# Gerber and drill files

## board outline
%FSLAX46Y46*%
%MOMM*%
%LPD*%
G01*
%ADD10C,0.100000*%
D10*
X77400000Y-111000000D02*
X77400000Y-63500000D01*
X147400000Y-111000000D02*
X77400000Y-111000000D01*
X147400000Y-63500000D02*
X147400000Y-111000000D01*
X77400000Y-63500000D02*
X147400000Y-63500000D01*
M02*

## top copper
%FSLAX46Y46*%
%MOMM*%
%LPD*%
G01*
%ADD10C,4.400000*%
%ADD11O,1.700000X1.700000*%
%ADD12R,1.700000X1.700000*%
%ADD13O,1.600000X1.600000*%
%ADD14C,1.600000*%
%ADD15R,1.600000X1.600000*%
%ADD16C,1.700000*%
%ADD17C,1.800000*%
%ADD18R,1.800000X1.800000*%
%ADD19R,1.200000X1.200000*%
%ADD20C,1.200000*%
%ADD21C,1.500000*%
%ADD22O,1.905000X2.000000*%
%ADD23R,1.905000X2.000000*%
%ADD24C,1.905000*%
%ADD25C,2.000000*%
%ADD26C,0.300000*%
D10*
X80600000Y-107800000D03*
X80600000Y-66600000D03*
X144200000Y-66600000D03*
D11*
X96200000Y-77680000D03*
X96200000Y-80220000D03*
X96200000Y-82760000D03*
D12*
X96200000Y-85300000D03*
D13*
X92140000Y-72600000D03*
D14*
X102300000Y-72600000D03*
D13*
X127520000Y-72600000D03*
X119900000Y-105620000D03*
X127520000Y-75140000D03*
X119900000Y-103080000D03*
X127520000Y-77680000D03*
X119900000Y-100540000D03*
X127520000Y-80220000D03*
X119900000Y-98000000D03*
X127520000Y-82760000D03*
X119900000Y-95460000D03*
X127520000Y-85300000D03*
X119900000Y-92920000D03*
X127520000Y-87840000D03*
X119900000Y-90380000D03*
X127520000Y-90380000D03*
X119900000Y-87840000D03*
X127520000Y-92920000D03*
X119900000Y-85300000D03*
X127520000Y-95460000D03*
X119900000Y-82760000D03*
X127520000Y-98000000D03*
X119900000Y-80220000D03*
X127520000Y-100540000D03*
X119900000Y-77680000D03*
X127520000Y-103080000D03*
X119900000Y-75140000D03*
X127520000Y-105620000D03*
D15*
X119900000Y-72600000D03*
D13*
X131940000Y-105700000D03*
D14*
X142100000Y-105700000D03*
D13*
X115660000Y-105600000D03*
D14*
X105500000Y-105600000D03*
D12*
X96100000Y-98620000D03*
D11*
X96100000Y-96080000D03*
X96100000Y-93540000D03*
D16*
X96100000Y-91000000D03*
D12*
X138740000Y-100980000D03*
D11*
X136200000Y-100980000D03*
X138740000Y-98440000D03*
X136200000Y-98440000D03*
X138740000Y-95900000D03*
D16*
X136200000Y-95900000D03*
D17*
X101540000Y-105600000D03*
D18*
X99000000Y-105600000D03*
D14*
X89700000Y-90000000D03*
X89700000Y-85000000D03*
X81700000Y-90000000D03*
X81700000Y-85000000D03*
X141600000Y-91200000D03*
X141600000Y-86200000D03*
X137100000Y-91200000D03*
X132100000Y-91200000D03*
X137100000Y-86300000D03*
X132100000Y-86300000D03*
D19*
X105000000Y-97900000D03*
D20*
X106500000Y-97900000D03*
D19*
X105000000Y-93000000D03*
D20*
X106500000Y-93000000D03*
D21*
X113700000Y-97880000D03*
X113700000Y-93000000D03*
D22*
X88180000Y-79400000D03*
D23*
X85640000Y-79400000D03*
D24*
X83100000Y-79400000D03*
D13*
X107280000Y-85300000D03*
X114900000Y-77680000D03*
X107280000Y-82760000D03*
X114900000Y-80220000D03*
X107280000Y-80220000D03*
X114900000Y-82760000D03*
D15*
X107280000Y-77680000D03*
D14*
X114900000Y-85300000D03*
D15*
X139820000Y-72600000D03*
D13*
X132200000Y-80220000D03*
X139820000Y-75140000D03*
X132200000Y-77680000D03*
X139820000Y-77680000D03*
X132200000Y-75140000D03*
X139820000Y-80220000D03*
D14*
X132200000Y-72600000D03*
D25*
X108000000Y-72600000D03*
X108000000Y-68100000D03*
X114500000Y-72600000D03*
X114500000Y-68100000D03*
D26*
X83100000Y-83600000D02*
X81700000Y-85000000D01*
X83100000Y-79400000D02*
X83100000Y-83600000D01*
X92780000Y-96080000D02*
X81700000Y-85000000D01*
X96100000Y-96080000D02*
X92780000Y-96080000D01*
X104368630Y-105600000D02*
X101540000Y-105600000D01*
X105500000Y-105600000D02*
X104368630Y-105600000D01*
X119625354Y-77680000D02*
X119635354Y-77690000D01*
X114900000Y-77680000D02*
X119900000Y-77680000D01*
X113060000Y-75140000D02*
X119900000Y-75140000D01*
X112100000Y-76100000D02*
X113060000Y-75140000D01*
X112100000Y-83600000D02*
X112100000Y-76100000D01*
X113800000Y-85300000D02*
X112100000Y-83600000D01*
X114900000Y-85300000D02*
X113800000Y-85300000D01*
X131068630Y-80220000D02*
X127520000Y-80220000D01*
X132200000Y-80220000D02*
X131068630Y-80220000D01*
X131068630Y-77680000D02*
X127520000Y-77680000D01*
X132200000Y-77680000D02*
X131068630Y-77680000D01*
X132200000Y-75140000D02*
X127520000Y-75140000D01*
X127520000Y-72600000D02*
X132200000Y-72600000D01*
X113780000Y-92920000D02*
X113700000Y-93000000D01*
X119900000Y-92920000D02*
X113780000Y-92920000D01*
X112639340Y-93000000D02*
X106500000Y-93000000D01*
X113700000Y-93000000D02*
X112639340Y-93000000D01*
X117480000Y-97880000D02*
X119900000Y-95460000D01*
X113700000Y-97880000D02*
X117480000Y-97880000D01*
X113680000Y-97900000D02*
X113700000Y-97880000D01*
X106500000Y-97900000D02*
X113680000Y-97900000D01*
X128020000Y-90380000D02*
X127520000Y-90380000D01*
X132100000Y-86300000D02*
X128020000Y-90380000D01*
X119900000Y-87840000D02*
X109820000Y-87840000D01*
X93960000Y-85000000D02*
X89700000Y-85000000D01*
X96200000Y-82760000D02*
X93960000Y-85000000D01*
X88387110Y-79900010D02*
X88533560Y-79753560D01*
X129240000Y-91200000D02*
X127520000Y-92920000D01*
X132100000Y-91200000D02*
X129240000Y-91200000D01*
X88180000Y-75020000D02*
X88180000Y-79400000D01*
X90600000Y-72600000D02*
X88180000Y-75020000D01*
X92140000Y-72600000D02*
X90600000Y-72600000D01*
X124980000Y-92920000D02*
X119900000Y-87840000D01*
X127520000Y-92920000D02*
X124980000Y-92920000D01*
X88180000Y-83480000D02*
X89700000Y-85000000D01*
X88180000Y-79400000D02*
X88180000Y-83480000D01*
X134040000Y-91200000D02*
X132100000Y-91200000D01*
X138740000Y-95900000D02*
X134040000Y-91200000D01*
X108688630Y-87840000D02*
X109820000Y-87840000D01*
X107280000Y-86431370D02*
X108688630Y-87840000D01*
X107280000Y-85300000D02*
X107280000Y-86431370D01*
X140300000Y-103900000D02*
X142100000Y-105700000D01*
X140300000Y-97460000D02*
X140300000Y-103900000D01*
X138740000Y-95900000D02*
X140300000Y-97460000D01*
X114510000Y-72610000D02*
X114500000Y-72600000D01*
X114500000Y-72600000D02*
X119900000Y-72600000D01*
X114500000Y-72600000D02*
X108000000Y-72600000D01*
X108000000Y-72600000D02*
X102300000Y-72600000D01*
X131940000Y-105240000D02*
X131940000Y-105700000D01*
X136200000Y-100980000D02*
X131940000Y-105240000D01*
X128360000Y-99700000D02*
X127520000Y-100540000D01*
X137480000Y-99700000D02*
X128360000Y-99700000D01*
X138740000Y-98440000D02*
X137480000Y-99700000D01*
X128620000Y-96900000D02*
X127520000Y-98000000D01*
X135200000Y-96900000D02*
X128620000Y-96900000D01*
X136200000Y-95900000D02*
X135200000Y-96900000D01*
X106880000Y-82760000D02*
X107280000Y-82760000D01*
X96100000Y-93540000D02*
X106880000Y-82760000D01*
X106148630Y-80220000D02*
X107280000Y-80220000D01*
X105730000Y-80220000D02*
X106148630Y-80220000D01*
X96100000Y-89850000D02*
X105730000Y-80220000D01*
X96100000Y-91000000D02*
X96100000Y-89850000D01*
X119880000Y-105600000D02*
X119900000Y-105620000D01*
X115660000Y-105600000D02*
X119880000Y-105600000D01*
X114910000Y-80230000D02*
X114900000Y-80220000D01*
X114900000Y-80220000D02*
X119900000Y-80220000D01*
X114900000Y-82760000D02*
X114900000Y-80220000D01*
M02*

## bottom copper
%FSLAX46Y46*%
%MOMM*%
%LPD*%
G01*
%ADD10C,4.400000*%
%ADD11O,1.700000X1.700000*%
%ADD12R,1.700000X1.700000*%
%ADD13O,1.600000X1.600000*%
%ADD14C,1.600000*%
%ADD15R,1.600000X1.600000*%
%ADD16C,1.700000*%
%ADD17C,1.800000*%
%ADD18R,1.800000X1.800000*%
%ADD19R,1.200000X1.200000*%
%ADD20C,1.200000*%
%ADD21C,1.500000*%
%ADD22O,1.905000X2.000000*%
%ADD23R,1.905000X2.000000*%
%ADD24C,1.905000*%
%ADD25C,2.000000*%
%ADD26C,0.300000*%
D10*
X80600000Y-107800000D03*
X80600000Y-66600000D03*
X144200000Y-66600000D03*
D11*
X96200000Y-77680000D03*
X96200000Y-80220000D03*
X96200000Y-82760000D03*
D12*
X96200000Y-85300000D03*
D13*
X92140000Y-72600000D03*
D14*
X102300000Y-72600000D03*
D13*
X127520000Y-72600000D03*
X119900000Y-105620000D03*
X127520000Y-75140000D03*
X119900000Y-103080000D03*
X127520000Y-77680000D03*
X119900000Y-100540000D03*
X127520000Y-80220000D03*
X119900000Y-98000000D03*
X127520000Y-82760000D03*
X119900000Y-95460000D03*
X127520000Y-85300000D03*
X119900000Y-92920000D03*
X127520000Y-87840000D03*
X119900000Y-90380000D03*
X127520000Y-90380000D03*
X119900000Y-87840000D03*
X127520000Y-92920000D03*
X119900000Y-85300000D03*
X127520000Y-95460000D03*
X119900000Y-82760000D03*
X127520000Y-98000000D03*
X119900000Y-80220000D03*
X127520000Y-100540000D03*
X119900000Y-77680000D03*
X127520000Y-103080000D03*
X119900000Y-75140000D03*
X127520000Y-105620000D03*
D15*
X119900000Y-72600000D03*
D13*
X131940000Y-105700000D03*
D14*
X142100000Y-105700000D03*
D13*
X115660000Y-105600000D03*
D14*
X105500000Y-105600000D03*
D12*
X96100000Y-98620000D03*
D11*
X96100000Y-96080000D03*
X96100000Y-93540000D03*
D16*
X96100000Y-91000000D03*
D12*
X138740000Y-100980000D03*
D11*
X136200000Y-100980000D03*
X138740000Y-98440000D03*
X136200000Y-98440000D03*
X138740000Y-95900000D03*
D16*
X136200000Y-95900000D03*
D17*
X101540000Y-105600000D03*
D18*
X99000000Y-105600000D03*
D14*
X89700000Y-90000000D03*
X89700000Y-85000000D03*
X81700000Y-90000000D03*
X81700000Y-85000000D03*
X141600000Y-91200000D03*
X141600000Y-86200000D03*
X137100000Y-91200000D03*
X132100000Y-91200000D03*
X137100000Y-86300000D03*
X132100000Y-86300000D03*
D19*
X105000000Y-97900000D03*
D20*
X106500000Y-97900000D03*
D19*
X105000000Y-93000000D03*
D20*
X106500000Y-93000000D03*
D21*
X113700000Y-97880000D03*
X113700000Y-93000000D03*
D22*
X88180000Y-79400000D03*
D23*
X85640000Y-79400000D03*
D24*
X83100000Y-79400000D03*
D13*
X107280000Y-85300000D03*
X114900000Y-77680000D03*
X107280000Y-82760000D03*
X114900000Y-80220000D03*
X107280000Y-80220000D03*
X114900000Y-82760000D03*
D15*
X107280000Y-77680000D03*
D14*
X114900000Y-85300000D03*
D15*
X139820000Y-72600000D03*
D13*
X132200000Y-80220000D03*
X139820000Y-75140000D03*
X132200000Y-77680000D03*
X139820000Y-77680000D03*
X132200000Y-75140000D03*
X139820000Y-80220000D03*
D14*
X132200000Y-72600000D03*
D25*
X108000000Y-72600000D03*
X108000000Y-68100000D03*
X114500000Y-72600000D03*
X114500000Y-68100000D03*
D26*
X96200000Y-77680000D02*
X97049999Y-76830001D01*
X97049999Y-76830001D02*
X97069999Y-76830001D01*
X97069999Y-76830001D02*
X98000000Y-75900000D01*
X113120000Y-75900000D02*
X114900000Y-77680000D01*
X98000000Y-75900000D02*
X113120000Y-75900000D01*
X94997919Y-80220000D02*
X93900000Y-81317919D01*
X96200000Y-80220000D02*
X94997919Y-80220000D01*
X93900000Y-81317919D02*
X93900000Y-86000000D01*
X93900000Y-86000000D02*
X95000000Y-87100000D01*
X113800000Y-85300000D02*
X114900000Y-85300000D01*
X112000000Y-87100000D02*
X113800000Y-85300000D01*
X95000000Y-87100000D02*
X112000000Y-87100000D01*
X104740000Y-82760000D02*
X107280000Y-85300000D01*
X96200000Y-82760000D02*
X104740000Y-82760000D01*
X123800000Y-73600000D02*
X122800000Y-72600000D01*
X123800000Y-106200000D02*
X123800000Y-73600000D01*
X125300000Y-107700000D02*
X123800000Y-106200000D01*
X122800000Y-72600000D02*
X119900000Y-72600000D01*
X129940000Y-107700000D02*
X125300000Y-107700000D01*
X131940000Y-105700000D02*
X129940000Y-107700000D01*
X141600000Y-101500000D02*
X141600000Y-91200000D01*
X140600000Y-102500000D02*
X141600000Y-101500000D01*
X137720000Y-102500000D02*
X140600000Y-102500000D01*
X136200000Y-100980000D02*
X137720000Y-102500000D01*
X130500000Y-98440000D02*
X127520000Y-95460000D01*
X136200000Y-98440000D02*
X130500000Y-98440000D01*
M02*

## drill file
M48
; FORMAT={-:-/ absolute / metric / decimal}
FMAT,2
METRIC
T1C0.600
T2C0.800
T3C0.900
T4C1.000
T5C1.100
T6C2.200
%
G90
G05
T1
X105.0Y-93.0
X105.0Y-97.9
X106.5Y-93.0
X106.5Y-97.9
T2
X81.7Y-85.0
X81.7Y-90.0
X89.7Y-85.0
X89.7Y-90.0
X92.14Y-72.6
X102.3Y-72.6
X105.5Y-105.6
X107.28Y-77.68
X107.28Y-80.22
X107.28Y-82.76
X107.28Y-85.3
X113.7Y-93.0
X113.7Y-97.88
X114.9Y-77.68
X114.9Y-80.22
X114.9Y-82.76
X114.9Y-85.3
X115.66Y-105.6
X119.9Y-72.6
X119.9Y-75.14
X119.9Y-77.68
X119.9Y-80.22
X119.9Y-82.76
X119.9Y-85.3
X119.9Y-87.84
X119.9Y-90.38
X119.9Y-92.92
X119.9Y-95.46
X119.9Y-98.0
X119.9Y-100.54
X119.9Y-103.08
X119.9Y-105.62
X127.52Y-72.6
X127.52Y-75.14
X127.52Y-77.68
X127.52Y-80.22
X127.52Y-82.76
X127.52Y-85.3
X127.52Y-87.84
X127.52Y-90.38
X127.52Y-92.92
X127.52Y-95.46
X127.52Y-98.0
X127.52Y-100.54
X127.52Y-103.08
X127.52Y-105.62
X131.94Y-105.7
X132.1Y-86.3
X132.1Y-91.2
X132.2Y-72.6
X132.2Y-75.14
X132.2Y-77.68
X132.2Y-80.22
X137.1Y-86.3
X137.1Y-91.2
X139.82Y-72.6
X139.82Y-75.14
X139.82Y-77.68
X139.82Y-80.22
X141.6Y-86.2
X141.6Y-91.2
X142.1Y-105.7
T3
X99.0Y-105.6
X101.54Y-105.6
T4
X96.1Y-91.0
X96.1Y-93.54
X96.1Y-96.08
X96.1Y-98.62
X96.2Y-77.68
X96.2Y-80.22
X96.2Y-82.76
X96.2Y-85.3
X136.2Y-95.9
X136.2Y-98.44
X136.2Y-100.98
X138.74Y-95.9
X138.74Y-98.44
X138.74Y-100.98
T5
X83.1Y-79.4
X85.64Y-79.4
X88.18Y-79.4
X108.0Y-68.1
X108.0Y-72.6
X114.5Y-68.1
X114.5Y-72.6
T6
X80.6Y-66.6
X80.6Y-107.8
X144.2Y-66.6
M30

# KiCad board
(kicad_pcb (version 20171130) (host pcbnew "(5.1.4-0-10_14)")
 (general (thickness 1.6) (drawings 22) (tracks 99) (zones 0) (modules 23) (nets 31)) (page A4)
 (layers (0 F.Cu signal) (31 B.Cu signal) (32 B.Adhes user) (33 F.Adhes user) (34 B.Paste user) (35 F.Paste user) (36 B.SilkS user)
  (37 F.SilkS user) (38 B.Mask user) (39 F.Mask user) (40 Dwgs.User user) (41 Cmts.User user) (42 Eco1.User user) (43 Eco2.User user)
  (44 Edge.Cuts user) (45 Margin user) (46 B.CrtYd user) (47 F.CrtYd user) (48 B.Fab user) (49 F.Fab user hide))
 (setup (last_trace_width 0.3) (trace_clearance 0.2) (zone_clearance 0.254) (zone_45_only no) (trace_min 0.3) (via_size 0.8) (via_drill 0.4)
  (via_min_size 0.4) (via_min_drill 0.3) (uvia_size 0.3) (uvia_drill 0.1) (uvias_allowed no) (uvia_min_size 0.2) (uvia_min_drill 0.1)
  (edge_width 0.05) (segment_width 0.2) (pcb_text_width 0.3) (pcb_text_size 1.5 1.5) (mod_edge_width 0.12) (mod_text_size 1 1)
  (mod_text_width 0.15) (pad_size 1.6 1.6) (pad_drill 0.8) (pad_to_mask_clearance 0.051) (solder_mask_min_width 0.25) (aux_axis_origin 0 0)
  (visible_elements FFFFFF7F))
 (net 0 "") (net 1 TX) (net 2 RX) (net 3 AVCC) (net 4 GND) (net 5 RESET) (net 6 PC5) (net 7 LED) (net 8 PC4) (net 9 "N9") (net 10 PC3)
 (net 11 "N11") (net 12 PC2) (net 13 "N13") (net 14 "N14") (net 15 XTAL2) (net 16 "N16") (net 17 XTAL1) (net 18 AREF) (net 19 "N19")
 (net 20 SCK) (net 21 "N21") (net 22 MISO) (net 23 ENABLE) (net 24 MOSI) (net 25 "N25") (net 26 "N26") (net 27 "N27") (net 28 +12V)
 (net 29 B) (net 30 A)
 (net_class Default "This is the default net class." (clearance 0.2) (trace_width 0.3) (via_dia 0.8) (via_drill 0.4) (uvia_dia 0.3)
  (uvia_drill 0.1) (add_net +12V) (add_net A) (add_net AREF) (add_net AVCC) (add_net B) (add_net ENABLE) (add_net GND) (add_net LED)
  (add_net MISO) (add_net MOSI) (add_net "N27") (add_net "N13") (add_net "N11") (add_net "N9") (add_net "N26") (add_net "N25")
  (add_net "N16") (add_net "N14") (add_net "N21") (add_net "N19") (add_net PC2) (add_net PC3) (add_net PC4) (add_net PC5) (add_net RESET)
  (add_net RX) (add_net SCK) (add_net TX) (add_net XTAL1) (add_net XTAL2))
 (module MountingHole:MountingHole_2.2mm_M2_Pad (layer F.Cu) (at 80.6 107.8)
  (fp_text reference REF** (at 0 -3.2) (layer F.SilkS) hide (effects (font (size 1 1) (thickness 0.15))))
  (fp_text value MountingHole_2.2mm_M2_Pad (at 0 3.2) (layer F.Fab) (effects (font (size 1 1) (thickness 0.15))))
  (pad 1 thru_hole circle (at 0 0) (size 4.4 4.4) (drill 2.2) (layers *.Cu *.Mask)))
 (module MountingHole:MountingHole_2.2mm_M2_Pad (layer F.Cu) (at 80.6 66.6)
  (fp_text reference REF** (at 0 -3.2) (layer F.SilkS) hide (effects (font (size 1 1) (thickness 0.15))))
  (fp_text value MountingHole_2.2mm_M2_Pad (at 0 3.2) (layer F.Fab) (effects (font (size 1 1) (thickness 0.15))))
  (pad 1 thru_hole circle (at 0 0) (size 4.4 4.4) (drill 2.2) (layers *.Cu *.Mask)))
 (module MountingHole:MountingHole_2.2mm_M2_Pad (layer F.Cu) (at 144.2 66.6)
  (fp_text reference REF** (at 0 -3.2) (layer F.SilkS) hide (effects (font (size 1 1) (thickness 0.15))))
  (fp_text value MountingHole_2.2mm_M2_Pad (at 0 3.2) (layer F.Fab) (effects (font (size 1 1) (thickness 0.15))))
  (pad 1 thru_hole circle (at 0 0) (size 4.4 4.4) (drill 2.2) (layers *.Cu *.Mask)))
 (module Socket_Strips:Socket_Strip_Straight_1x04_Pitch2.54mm (layer F.Cu) (at 96.2 85.3 180)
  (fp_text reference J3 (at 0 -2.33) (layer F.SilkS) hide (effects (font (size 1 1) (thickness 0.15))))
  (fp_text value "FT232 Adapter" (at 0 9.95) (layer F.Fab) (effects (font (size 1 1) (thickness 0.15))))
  (pad 4 thru_hole oval (at 0 7.62 180) (size 1.7 1.7) (drill 1) (layers *.Cu *.Mask) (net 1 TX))
  (pad 3 thru_hole oval (at 0 5.08 180) (size 1.7 1.7) (drill 1) (layers *.Cu *.Mask) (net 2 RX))
  (pad 2 thru_hole oval (at 0 2.54 180) (size 1.7 1.7) (drill 1) (layers *.Cu *.Mask) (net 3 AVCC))
  (pad 1 thru_hole rect (at 0 0 180) (size 1.7 1.7) (drill 1) (layers *.Cu *.Mask) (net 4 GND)))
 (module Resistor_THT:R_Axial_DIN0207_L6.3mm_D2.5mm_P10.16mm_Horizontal (layer F.Cu) (at 102.3 72.6 180)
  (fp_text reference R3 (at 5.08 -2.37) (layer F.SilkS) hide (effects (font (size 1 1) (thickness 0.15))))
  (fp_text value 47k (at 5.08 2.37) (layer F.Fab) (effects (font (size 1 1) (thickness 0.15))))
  (pad 2 thru_hole oval (at 10.16 0 180) (size 1.6 1.6) (drill 0.8) (layers *.Cu *.Mask) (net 3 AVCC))
  (pad 1 thru_hole circle (at 0 0 180) (size 1.6 1.6) (drill 0.8) (layers *.Cu *.Mask) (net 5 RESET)))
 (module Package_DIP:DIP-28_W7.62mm (layer F.Cu) (at 119.9 72.6)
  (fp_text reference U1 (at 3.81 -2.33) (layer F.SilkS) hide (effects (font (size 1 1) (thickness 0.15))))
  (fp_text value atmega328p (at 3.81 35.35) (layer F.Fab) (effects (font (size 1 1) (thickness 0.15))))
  (pad 28 thru_hole oval (at 7.62 0) (size 1.6 1.6) (drill 0.8) (layers *.Cu *.Mask) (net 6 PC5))
  (pad 14 thru_hole oval (at 0 33.02) (size 1.6 1.6) (drill 0.8) (layers *.Cu *.Mask) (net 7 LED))
  (pad 27 thru_hole oval (at 7.62 2.54) (size 1.6 1.6) (drill 0.8) (layers *.Cu *.Mask) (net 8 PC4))
  (pad 13 thru_hole oval (at 0 30.48) (size 1.6 1.6) (drill 0.8) (layers *.Cu *.Mask) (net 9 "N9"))
  (pad 26 thru_hole oval (at 7.62 5.08) (size 1.6 1.6) (drill 0.8) (layers *.Cu *.Mask) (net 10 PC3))
  (pad 12 thru_hole oval (at 0 27.94) (size 1.6 1.6) (drill 0.8) (layers *.Cu *.Mask) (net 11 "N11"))
  (pad 25 thru_hole oval (at 7.62 7.62) (size 1.6 1.6) (drill 0.8) (layers *.Cu *.Mask) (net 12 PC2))
  (pad 11 thru_hole oval (at 0 25.4) (size 1.6 1.6) (drill 0.8) (layers *.Cu *.Mask) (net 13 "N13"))
  (pad 24 thru_hole oval (at 7.62 10.16) (size 1.6 1.6) (drill 0.8) (layers *.Cu *.Mask) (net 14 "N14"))
  (pad 10 thru_hole oval (at 0 22.86) (size 1.6 1.6) (drill 0.8) (layers *.Cu *.Mask) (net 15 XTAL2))
  (pad 23 thru_hole oval (at 7.62 12.7) (size 1.6 1.6) (drill 0.8) (layers *.Cu *.Mask) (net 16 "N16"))
  (pad 9 thru_hole oval (at 0 20.32) (size 1.6 1.6) (drill 0.8) (layers *.Cu *.Mask) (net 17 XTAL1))
  (pad 22 thru_hole oval (at 7.62 15.24) (size 1.6 1.6) (drill 0.8) (layers *.Cu *.Mask) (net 4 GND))
  (pad 8 thru_hole oval (at 0 17.78) (size 1.6 1.6) (drill 0.8) (layers *.Cu *.Mask) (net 4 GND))
  (pad 21 thru_hole oval (at 7.62 17.78) (size 1.6 1.6) (drill 0.8) (layers *.Cu *.Mask) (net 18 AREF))
  (pad 7 thru_hole oval (at 0 15.24) (size 1.6 1.6) (drill 0.8) (layers *.Cu *.Mask) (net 3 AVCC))
  (pad 20 thru_hole oval (at 7.62 20.32) (size 1.6 1.6) (drill 0.8) (layers *.Cu *.Mask) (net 3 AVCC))
  (pad 6 thru_hole oval (at 0 12.7) (size 1.6 1.6) (drill 0.8) (layers *.Cu *.Mask) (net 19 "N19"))
  (pad 19 thru_hole oval (at 7.62 22.86) (size 1.6 1.6) (drill 0.8) (layers *.Cu *.Mask) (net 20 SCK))
  (pad 5 thru_hole oval (at 0 10.16) (size 1.6 1.6) (drill 0.8) (layers *.Cu *.Mask) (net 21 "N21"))
  (pad 18 thru_hole oval (at 7.62 25.4) (size 1.6 1.6) (drill 0.8) (layers *.Cu *.Mask) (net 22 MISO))
  (pad 4 thru_hole oval (at 0 7.62) (size 1.6 1.6) (drill 0.8) (layers *.Cu *.Mask) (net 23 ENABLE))
  (pad 17 thru_hole oval (at 7.62 27.94) (size 1.6 1.6) (drill 0.8) (layers *.Cu *.Mask) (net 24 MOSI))
  (pad 3 thru_hole oval (at 0 5.08) (size 1.6 1.6) (drill 0.8) (layers *.Cu *.Mask) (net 1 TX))
  (pad 16 thru_hole oval (at 7.62 30.48) (size 1.6 1.6) (drill 0.8) (layers *.Cu *.Mask) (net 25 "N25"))
  (pad 2 thru_hole oval (at 0 2.54) (size 1.6 1.6) (drill 0.8) (layers *.Cu *.Mask) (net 2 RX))
  (pad 15 thru_hole oval (at 7.62 33.02) (size 1.6 1.6) (drill 0.8) (layers *.Cu *.Mask) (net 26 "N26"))
  (pad 1 thru_hole rect (at 0 0) (size 1.6 1.6) (drill 0.8) (layers *.Cu *.Mask) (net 5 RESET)))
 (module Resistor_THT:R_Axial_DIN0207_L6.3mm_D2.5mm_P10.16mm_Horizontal (layer F.Cu) (at 142.1 105.7 180)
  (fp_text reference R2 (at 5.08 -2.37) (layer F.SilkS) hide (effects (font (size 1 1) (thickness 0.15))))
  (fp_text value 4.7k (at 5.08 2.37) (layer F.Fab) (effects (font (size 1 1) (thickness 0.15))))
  (pad 2 thru_hole oval (at 10.16 0 180) (size 1.6 1.6) (drill 0.8) (layers *.Cu *.Mask) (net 5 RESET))
  (pad 1 thru_hole circle (at 0 0 180) (size 1.6 1.6) (drill 0.8) (layers *.Cu *.Mask) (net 3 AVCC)))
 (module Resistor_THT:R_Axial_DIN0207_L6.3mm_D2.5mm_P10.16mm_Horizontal (layer F.Cu) (at 105.5 105.6)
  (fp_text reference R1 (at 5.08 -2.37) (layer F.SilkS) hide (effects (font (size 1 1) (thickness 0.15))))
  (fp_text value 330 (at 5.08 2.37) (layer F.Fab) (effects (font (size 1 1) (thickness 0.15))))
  (pad 2 thru_hole oval (at 10.16 0) (size 1.6 1.6) (drill 0.8) (layers *.Cu *.Mask) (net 7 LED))
  (pad 1 thru_hole circle (at 0 0) (size 1.6 1.6) (drill 0.8) (layers *.Cu *.Mask) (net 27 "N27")))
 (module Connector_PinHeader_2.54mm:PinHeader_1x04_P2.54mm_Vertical (layer F.Cu) (at 96.1 91)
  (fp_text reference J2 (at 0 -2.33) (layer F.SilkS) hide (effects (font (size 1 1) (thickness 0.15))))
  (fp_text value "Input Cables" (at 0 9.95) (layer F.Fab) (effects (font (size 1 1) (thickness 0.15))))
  (pad 4 thru_hole rect (at 0 7.62) (size 1.7 1.7) (drill 1) (layers *.Cu *.Mask) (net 4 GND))
  (pad 3 thru_hole oval (at 0 5.08) (size 1.7 1.7) (drill 1) (layers *.Cu *.Mask) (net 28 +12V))
  (pad 2 thru_hole oval (at 0 2.54) (size 1.7 1.7) (drill 1) (layers *.Cu *.Mask) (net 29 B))
  (pad 1 thru_hole circle (at 0 0) (size 1.7 1.7) (drill 1) (layers *.Cu *.Mask) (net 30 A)))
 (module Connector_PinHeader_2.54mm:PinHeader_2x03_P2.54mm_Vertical (layer F.Cu) (at 136.2 95.9)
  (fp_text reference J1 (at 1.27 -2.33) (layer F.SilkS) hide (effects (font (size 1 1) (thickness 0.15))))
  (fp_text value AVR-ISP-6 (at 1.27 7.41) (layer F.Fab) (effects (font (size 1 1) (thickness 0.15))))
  (pad 6 thru_hole rect (at 2.54 5.08) (size 1.7 1.7) (drill 1) (layers *.Cu *.Mask) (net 4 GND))
  (pad 5 thru_hole oval (at 0 5.08) (size 1.7 1.7) (drill 1) (layers *.Cu *.Mask) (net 5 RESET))
  (pad 4 thru_hole oval (at 2.54 2.54) (size 1.7 1.7) (drill 1) (layers *.Cu *.Mask) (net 24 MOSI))
  (pad 3 thru_hole oval (at 0 2.54) (size 1.7 1.7) (drill 1) (layers *.Cu *.Mask) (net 20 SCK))
  (pad 2 thru_hole oval (at 2.54 0) (size 1.7 1.7) (drill 1) (layers *.Cu *.Mask) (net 3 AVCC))
  (pad 1 thru_hole circle (at 0 0) (size 1.7 1.7) (drill 1) (layers *.Cu *.Mask) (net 22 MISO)))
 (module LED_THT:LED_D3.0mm (layer F.Cu) (at 99 105.6)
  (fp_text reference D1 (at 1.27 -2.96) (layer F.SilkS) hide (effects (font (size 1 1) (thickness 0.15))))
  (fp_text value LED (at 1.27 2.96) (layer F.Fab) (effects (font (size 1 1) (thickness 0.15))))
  (pad 2 thru_hole circle (at 2.54 0) (size 1.8 1.8) (drill 0.9) (layers *.Cu *.Mask) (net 27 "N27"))
  (pad 1 thru_hole rect (at 0 0) (size 1.8 1.8) (drill 0.9) (layers *.Cu *.Mask) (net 4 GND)))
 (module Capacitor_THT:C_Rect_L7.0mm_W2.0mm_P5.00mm (layer F.Cu) (at 89.7 85 270)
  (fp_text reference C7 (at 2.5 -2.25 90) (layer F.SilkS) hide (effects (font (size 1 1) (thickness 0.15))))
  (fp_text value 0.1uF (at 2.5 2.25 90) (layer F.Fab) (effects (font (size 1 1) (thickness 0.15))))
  (pad 2 thru_hole circle (at 5 0 270) (size 1.6 1.6) (drill 0.8) (layers *.Cu *.Mask) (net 4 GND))
  (pad 1 thru_hole circle (at 0 0 270) (size 1.6 1.6) (drill 0.8) (layers *.Cu *.Mask) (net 3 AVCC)))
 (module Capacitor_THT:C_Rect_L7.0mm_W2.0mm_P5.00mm (layer F.Cu) (at 81.7 85 270)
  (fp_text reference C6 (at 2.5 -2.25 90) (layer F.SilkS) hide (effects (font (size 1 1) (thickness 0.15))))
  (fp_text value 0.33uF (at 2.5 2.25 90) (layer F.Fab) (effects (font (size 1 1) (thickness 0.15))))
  (pad 2 thru_hole circle (at 5 0 270) (size 1.6 1.6) (drill 0.8) (layers *.Cu *.Mask) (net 4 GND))
  (pad 1 thru_hole circle (at 0 0 270) (size 1.6 1.6) (drill 0.8) (layers *.Cu *.Mask) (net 28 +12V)))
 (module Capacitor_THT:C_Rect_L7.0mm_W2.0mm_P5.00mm (layer F.Cu) (at 141.6 86.2 270)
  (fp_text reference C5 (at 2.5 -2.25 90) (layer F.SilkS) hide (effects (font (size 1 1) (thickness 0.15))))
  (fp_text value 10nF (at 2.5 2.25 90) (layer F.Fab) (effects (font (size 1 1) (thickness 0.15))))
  (pad 2 thru_hole circle (at 5 0 270) (size 1.6 1.6) (drill 0.8) (layers *.Cu *.Mask) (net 5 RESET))
  (pad 1 thru_hole circle (at 0 0 270) (size 1.6 1.6) (drill 0.8) (layers *.Cu *.Mask) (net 4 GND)))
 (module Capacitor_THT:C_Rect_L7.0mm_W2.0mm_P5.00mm (layer F.Cu) (at 132.1 91.2)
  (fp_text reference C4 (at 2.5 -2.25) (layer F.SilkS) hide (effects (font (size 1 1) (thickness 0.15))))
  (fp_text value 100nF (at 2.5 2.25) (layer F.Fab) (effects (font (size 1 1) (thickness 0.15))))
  (pad 2 thru_hole circle (at 5 0) (size 1.6 1.6) (drill 0.8) (layers *.Cu *.Mask) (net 4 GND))
  (pad 1 thru_hole circle (at 0 0) (size 1.6 1.6) (drill 0.8) (layers *.Cu *.Mask) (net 3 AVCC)))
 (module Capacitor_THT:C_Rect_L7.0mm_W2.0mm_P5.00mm (layer F.Cu) (at 132.1 86.3)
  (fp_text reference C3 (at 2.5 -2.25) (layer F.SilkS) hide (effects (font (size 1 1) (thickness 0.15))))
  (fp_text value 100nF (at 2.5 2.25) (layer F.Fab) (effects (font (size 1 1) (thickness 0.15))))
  (pad 2 thru_hole circle (at 5 0) (size 1.6 1.6) (drill 0.8) (layers *.Cu *.Mask) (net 4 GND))
  (pad 1 thru_hole circle (at 0 0) (size 1.6 1.6) (drill 0.8) (layers *.Cu *.Mask) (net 18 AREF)))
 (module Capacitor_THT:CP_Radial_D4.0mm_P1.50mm (layer F.Cu) (at 106.5 97.9 180)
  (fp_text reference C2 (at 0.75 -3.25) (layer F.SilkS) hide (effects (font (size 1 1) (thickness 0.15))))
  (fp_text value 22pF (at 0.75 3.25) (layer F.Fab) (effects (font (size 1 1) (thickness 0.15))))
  (pad 2 thru_hole rect (at 1.5 0 180) (size 1.2 1.2) (drill 0.6) (layers *.Cu *.Mask) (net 4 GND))
  (pad 1 thru_hole circle (at 0 0 180) (size 1.2 1.2) (drill 0.6) (layers *.Cu *.Mask) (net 15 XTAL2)))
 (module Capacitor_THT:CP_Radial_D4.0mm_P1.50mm (layer F.Cu) (at 106.5 93 180)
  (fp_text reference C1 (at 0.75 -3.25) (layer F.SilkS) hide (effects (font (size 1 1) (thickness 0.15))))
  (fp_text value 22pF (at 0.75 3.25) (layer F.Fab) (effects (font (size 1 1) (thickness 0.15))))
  (pad 2 thru_hole rect (at 1.5 0 180) (size 1.2 1.2) (drill 0.6) (layers *.Cu *.Mask) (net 4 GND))
  (pad 1 thru_hole circle (at 0 0 180) (size 1.2 1.2) (drill 0.6) (layers *.Cu *.Mask) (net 17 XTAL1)))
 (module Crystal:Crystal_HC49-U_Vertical (layer F.Cu) (at 113.7 93 270)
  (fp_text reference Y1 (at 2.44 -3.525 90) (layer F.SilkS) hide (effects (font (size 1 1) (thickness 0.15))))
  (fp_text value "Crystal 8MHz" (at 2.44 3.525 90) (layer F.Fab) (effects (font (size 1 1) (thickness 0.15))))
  (pad 2 thru_hole circle (at 4.88 0 270) (size 1.5 1.5) (drill 0.8) (layers *.Cu *.Mask) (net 15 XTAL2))
  (pad 1 thru_hole circle (at 0 0 270) (size 1.5 1.5) (drill 0.8) (layers *.Cu *.Mask) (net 17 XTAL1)))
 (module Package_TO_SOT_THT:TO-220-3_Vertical (layer F.Cu) (at 83.1 79.4)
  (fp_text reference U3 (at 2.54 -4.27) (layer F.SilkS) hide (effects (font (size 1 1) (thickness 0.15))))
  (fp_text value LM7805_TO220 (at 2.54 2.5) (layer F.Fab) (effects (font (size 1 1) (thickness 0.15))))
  (pad 3 thru_hole oval (at 5.08 0) (size 1.905 2) (drill 1.1) (layers *.Cu *.Mask) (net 3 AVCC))
  (pad 2 thru_hole rect (at 2.54 0) (size 1.905 2) (drill 1.1) (layers *.Cu *.Mask) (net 4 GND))
  (pad 1 thru_hole circle (at 0 0) (size 1.905 1.905) (drill 1.1) (layers *.Cu *.Mask) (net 28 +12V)))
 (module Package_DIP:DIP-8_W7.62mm (layer F.Cu) (at 114.9 85.3 180)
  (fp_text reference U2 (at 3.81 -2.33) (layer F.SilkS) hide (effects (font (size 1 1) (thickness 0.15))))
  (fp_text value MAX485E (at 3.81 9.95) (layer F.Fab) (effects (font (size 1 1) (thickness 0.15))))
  (pad 8 thru_hole oval (at 7.62 0 180) (size 1.6 1.6) (drill 0.8) (layers *.Cu *.Mask) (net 3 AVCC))
  (pad 4 thru_hole oval (at 0 7.62 180) (size 1.6 1.6) (drill 0.8) (layers *.Cu *.Mask) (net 1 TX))
  (pad 7 thru_hole oval (at 7.62 2.54 180) (size 1.6 1.6) (drill 0.8) (layers *.Cu *.Mask) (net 29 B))
  (pad 3 thru_hole oval (at 0 5.08 180) (size 1.6 1.6) (drill 0.8) (layers *.Cu *.Mask) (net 23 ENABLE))
  (pad 6 thru_hole oval (at 7.62 5.08 180) (size 1.6 1.6) (drill 0.8) (layers *.Cu *.Mask) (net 30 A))
  (pad 2 thru_hole oval (at 0 2.54 180) (size 1.6 1.6) (drill 0.8) (layers *.Cu *.Mask) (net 23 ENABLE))
  (pad 5 thru_hole rect (at 7.62 7.62 180) (size 1.6 1.6) (drill 0.8) (layers *.Cu *.Mask) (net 4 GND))
  (pad 1 thru_hole circle (at 0 0 180) (size 1.6 1.6) (drill 0.8) (layers *.Cu *.Mask) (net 2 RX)))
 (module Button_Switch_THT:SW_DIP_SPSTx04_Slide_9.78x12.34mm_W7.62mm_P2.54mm (layer F.Cu) (at 132.2 72.6)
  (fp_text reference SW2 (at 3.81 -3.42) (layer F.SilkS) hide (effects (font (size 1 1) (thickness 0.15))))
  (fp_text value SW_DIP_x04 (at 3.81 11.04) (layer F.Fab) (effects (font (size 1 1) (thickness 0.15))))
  (pad 8 thru_hole rect (at 7.62 0) (size 1.6 1.6) (drill 0.8) (layers *.Cu *.Mask) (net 4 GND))
  (pad 4 thru_hole oval (at 0 7.62) (size 1.6 1.6) (drill 0.8) (layers *.Cu *.Mask) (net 12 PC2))
  (pad 7 thru_hole oval (at 7.62 2.54) (size 1.6 1.6) (drill 0.8) (layers *.Cu *.Mask) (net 4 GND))
  (pad 3 thru_hole oval (at 0 5.08) (size 1.6 1.6) (drill 0.8) (layers *.Cu *.Mask) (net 10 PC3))
  (pad 6 thru_hole oval (at 7.62 5.08) (size 1.6 1.6) (drill 0.8) (layers *.Cu *.Mask) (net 4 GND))
  (pad 2 thru_hole oval (at 0 2.54) (size 1.6 1.6) (drill 0.8) (layers *.Cu *.Mask) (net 8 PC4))
  (pad 5 thru_hole oval (at 7.62 7.62) (size 1.6 1.6) (drill 0.8) (layers *.Cu *.Mask) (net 4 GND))
  (pad 1 thru_hole circle (at 0 0) (size 1.6 1.6) (drill 0.8) (layers *.Cu *.Mask) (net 6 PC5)))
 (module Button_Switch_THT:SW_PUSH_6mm (layer F.Cu) (at 114.5 72.6 180)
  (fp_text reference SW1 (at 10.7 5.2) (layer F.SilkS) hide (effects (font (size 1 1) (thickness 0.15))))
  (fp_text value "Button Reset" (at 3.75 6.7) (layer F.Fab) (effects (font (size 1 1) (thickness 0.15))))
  (pad 1 thru_hole circle (at 6.5 0 270) (size 2 2) (drill 1.1) (layers *.Cu *.Mask) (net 5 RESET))
  (pad 2 thru_hole circle (at 6.5 4.5 270) (size 2 2) (drill 1.1) (layers *.Cu *.Mask) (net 4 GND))
  (pad 1 thru_hole circle (at 0 0 270) (size 2 2) (drill 1.1) (layers *.Cu *.Mask) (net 5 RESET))
  (pad 2 thru_hole circle (at 0 4.5 270) (size 2 2) (drill 1.1) (layers *.Cu *.Mask) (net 4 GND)))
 (gr_line (start 77.4 111) (end 77.4 63.5) (layer Edge.Cuts) (width 0.1))
 (gr_line (start 147.4 111) (end 77.4 111) (layer Edge.Cuts) (width 0.1))
 (gr_line (start 147.4 63.5) (end 147.4 111) (layer Edge.Cuts) (width 0.1))
 (gr_line (start 77.4 63.5) (end 147.4 63.5) (layer Edge.Cuts) (width 0.1))
 (segment (start 83.1 83.6) (end 81.7 85) (width 0.3) (layer F.Cu) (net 28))
 (segment (start 83.1 79.4) (end 83.1 83.6) (width 0.3) (layer F.Cu) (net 28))
 (segment (start 92.78 96.08) (end 81.7 85) (width 0.3) (layer F.Cu) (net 28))
 (segment (start 96.1 96.08) (end 92.78 96.08) (width 0.3) (layer F.Cu) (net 28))
 (segment (start 104.36863 105.6) (end 101.54 105.6) (width 0.3) (layer F.Cu) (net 27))
 (segment (start 105.5 105.6) (end 104.36863 105.6) (width 0.3) (layer F.Cu) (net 27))
 (segment (start 119.625354 77.68) (end 119.635354 77.69) (width 0.3) (layer F.Cu) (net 1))
 (segment (start 114.9 77.68) (end 119.9 77.68) (width 0.3) (layer F.Cu) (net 1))
 (segment (start 96.2 77.68) (end 97.049999 76.830001) (width 0.3) (layer B.Cu) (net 1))
 (segment (start 97.049999 76.830001) (end 97.069999 76.830001) (width 0.3) (layer B.Cu) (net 1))
 (segment (start 97.069999 76.830001) (end 98 75.9) (width 0.3) (layer B.Cu) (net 1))
 (segment (start 113.12 75.9) (end 114.9 77.68) (width 0.3) (layer B.Cu) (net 1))
 (segment (start 98 75.9) (end 113.12 75.9) (width 0.3) (layer B.Cu) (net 1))
 (segment (start 113.06 75.14) (end 119.9 75.14) (width 0.3) (layer F.Cu) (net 2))
 (segment (start 112.1 76.1) (end 113.06 75.14) (width 0.3) (layer F.Cu) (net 2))
 (segment (start 112.1 83.6) (end 112.1 76.1) (width 0.3) (layer F.Cu) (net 2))
 (segment (start 113.8 85.3) (end 112.1 83.6) (width 0.3) (layer F.Cu) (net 2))
 (segment (start 114.9 85.3) (end 113.8 85.3) (width 0.3) (layer F.Cu) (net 2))
 (segment (start 94.997919 80.22) (end 93.9 81.317919) (width 0.3) (layer B.Cu) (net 2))
 (segment (start 96.2 80.22) (end 94.997919 80.22) (width 0.3) (layer B.Cu) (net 2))
 (segment (start 93.9 81.317919) (end 93.9 86) (width 0.3) (layer B.Cu) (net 2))
 (segment (start 93.9 86) (end 95 87.1) (width 0.3) (layer B.Cu) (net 2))
 (segment (start 113.8 85.3) (end 114.9 85.3) (width 0.3) (layer B.Cu) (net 2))
 (segment (start 112 87.1) (end 113.8 85.3) (width 0.3) (layer B.Cu) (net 2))
 (segment (start 95 87.1) (end 112 87.1) (width 0.3) (layer B.Cu) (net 2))
 (segment (start 131.06863 80.22) (end 127.52 80.22) (width 0.3) (layer F.Cu) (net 12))
 (segment (start 132.2 80.22) (end 131.06863 80.22) (width 0.3) (layer F.Cu) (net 12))
 (segment (start 131.06863 77.68) (end 127.52 77.68) (width 0.3) (layer F.Cu) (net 10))
 (segment (start 132.2 77.68) (end 131.06863 77.68) (width 0.3) (layer F.Cu) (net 10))
 (segment (start 132.2 75.14) (end 127.52 75.14) (width 0.3) (layer F.Cu) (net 8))
 (segment (start 127.52 72.6) (end 132.2 72.6) (width 0.3) (layer F.Cu) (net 6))
 (segment (start 113.78 92.92) (end 113.7 93) (width 0.3) (layer F.Cu) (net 17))
 (segment (start 119.9 92.92) (end 113.78 92.92) (width 0.3) (layer F.Cu) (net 17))
 (segment (start 112.63934 93) (end 106.5 93) (width 0.3) (layer F.Cu) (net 17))
 (segment (start 113.7 93) (end 112.63934 93) (width 0.3) (layer F.Cu) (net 17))
 (segment (start 117.48 97.88) (end 119.9 95.46) (width 0.3) (layer F.Cu) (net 15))
 (segment (start 113.7 97.88) (end 117.48 97.88) (width 0.3) (layer F.Cu) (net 15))
 (segment (start 113.68 97.9) (end 113.7 97.88) (width 0.3) (layer F.Cu) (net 15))
 (segment (start 106.5 97.9) (end 113.68 97.9) (width 0.3) (layer F.Cu) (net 15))
 (segment (start 128.02 90.38) (end 127.52 90.38) (width 0.3) (layer F.Cu) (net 18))
 (segment (start 132.1 86.3) (end 128.02 90.38) (width 0.3) (layer F.Cu) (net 18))
 (segment (start 119.9 87.84) (end 109.82 87.84) (width 0.3) (layer F.Cu) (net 3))
 (segment (start 93.96 85) (end 89.7 85) (width 0.3) (layer F.Cu) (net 3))
 (segment (start 96.2 82.76) (end 93.96 85) (width 0.3) (layer F.Cu) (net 3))
 (segment (start 88.38711 79.90001) (end 88.53356 79.75356) (width 0.3) (layer F.Cu) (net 3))
 (segment (start 129.24 91.2) (end 127.52 92.92) (width 0.3) (layer F.Cu) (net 3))
 (segment (start 132.1 91.2) (end 129.24 91.2) (width 0.3) (layer F.Cu) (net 3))
 (segment (start 88.18 75.02) (end 88.18 79.4) (width 0.3) (layer F.Cu) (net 3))
 (segment (start 90.6 72.6) (end 88.18 75.02) (width 0.3) (layer F.Cu) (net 3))
 (segment (start 92.14 72.6) (end 90.6 72.6) (width 0.3) (layer F.Cu) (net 3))
 (segment (start 124.98 92.92) (end 119.9 87.84) (width 0.3) (layer F.Cu) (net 3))
 (segment (start 127.52 92.92) (end 124.98 92.92) (width 0.3) (layer F.Cu) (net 3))
 (segment (start 104.74 82.76) (end 107.28 85.3) (width 0.3) (layer B.Cu) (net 3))
 (segment (start 96.2 82.76) (end 104.74 82.76) (width 0.3) (layer B.Cu) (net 3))
 (segment (start 88.18 83.48) (end 89.7 85) (width 0.3) (layer F.Cu) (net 3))
 (segment (start 88.18 79.4) (end 88.18 83.48) (width 0.3) (layer F.Cu) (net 3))
 (segment (start 134.04 91.2) (end 132.1 91.2) (width 0.3) (layer F.Cu) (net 3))
 (segment (start 138.74 95.9) (end 134.04 91.2) (width 0.3) (layer F.Cu) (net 3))
 (segment (start 108.68863 87.84) (end 109.82 87.84) (width 0.3) (layer F.Cu) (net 3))
 (segment (start 107.28 86.43137) (end 108.68863 87.84) (width 0.3) (layer F.Cu) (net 3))
 (segment (start 107.28 85.3) (end 107.28 86.43137) (width 0.3) (layer F.Cu) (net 3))
 (segment (start 140.3 103.9) (end 142.1 105.7) (width 0.3) (layer F.Cu) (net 3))
 (segment (start 140.3 97.46) (end 140.3 103.9) (width 0.3) (layer F.Cu) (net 3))
 (segment (start 138.74 95.9) (end 140.3 97.46) (width 0.3) (layer F.Cu) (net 3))
 (segment (start 114.51 72.61) (end 114.5 72.6) (width 0.3) (layer F.Cu) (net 5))
 (segment (start 114.5 72.6) (end 119.9 72.6) (width 0.3) (layer F.Cu) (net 5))
 (segment (start 114.5 72.6) (end 108 72.6) (width 0.3) (layer F.Cu) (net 5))
 (segment (start 108 72.6) (end 102.3 72.6) (width 0.3) (layer F.Cu) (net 5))
 (segment (start 123.8 73.6) (end 122.8 72.6) (width 0.3) (layer B.Cu) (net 5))
 (segment (start 123.8 106.2) (end 123.8 73.6) (width 0.3) (layer B.Cu) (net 5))
 (segment (start 125.3 107.7) (end 123.8 106.2) (width 0.3) (layer B.Cu) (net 5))
 (segment (start 122.8 72.6) (end 119.9 72.6) (width 0.3) (layer B.Cu) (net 5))
 (segment (start 131.94 105.24) (end 131.94 105.7) (width 0.3) (layer F.Cu) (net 5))
 (segment (start 136.2 100.98) (end 131.94 105.24) (width 0.3) (layer F.Cu) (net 5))
 (segment (start 129.94 107.7) (end 125.3 107.7) (width 0.3) (layer B.Cu) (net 5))
 (segment (start 131.94 105.7) (end 129.94 107.7) (width 0.3) (layer B.Cu) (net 5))
 (segment (start 141.6 101.5) (end 141.6 91.2) (width 0.3) (layer B.Cu) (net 5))
 (segment (start 140.6 102.5) (end 141.6 101.5) (width 0.3) (layer B.Cu) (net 5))
 (segment (start 137.72 102.5) (end 140.6 102.5) (width 0.3) (layer B.Cu) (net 5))
 (segment (start 136.2 100.98) (end 137.72 102.5) (width 0.3) (layer B.Cu) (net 5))
 (segment (start 128.36 99.7) (end 127.52 100.54) (width 0.3) (layer F.Cu) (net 24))
 (segment (start 137.48 99.7) (end 128.36 99.7) (width 0.3) (layer F.Cu) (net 24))
 (segment (start 138.74 98.44) (end 137.48 99.7) (width 0.3) (layer F.Cu) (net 24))
 (segment (start 130.5 98.44) (end 127.52 95.46) (width 0.3) (layer B.Cu) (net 20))
 (segment (start 136.2 98.44) (end 130.5 98.44) (width 0.3) (layer B.Cu) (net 20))
 (segment (start 128.62 96.9) (end 127.52 98) (width 0.3) (layer F.Cu) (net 22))
 (segment (start 135.2 96.9) (end 128.62 96.9) (width 0.3) (layer F.Cu) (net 22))
 (segment (start 136.2 95.9) (end 135.2 96.9) (width 0.3) (layer F.Cu) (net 22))
 (segment (start 106.88 82.76) (end 107.28 82.76) (width 0.3) (layer F.Cu) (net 29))
 (segment (start 96.1 93.54) (end 106.88 82.76) (width 0.3) (layer F.Cu) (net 29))
 (segment (start 106.14863 80.22) (end 107.28 80.22) (width 0.3) (layer F.Cu) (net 30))
 (segment (start 105.73 80.22) (end 106.14863 80.22) (width 0.3) (layer F.Cu) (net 30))
 (segment (start 96.1 89.85) (end 105.73 80.22) (width 0.3) (layer F.Cu) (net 30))
 (segment (start 96.1 91) (end 96.1 89.85) (width 0.3) (layer F.Cu) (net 30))
 (segment (start 119.88 105.6) (end 119.9 105.62) (width 0.3) (layer F.Cu) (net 7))
 (segment (start 115.66 105.6) (end 119.88 105.6) (width 0.3) (layer F.Cu) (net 7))
 (segment (start 114.91 80.23) (end 114.9 80.22) (width 0.3) (layer F.Cu) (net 23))
 (segment (start 114.9 80.22) (end 119.9 80.22) (width 0.3) (layer F.Cu) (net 23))
 (segment (start 114.9 82.76) (end 114.9 80.22) (width 0.3) (layer F.Cu) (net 23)))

